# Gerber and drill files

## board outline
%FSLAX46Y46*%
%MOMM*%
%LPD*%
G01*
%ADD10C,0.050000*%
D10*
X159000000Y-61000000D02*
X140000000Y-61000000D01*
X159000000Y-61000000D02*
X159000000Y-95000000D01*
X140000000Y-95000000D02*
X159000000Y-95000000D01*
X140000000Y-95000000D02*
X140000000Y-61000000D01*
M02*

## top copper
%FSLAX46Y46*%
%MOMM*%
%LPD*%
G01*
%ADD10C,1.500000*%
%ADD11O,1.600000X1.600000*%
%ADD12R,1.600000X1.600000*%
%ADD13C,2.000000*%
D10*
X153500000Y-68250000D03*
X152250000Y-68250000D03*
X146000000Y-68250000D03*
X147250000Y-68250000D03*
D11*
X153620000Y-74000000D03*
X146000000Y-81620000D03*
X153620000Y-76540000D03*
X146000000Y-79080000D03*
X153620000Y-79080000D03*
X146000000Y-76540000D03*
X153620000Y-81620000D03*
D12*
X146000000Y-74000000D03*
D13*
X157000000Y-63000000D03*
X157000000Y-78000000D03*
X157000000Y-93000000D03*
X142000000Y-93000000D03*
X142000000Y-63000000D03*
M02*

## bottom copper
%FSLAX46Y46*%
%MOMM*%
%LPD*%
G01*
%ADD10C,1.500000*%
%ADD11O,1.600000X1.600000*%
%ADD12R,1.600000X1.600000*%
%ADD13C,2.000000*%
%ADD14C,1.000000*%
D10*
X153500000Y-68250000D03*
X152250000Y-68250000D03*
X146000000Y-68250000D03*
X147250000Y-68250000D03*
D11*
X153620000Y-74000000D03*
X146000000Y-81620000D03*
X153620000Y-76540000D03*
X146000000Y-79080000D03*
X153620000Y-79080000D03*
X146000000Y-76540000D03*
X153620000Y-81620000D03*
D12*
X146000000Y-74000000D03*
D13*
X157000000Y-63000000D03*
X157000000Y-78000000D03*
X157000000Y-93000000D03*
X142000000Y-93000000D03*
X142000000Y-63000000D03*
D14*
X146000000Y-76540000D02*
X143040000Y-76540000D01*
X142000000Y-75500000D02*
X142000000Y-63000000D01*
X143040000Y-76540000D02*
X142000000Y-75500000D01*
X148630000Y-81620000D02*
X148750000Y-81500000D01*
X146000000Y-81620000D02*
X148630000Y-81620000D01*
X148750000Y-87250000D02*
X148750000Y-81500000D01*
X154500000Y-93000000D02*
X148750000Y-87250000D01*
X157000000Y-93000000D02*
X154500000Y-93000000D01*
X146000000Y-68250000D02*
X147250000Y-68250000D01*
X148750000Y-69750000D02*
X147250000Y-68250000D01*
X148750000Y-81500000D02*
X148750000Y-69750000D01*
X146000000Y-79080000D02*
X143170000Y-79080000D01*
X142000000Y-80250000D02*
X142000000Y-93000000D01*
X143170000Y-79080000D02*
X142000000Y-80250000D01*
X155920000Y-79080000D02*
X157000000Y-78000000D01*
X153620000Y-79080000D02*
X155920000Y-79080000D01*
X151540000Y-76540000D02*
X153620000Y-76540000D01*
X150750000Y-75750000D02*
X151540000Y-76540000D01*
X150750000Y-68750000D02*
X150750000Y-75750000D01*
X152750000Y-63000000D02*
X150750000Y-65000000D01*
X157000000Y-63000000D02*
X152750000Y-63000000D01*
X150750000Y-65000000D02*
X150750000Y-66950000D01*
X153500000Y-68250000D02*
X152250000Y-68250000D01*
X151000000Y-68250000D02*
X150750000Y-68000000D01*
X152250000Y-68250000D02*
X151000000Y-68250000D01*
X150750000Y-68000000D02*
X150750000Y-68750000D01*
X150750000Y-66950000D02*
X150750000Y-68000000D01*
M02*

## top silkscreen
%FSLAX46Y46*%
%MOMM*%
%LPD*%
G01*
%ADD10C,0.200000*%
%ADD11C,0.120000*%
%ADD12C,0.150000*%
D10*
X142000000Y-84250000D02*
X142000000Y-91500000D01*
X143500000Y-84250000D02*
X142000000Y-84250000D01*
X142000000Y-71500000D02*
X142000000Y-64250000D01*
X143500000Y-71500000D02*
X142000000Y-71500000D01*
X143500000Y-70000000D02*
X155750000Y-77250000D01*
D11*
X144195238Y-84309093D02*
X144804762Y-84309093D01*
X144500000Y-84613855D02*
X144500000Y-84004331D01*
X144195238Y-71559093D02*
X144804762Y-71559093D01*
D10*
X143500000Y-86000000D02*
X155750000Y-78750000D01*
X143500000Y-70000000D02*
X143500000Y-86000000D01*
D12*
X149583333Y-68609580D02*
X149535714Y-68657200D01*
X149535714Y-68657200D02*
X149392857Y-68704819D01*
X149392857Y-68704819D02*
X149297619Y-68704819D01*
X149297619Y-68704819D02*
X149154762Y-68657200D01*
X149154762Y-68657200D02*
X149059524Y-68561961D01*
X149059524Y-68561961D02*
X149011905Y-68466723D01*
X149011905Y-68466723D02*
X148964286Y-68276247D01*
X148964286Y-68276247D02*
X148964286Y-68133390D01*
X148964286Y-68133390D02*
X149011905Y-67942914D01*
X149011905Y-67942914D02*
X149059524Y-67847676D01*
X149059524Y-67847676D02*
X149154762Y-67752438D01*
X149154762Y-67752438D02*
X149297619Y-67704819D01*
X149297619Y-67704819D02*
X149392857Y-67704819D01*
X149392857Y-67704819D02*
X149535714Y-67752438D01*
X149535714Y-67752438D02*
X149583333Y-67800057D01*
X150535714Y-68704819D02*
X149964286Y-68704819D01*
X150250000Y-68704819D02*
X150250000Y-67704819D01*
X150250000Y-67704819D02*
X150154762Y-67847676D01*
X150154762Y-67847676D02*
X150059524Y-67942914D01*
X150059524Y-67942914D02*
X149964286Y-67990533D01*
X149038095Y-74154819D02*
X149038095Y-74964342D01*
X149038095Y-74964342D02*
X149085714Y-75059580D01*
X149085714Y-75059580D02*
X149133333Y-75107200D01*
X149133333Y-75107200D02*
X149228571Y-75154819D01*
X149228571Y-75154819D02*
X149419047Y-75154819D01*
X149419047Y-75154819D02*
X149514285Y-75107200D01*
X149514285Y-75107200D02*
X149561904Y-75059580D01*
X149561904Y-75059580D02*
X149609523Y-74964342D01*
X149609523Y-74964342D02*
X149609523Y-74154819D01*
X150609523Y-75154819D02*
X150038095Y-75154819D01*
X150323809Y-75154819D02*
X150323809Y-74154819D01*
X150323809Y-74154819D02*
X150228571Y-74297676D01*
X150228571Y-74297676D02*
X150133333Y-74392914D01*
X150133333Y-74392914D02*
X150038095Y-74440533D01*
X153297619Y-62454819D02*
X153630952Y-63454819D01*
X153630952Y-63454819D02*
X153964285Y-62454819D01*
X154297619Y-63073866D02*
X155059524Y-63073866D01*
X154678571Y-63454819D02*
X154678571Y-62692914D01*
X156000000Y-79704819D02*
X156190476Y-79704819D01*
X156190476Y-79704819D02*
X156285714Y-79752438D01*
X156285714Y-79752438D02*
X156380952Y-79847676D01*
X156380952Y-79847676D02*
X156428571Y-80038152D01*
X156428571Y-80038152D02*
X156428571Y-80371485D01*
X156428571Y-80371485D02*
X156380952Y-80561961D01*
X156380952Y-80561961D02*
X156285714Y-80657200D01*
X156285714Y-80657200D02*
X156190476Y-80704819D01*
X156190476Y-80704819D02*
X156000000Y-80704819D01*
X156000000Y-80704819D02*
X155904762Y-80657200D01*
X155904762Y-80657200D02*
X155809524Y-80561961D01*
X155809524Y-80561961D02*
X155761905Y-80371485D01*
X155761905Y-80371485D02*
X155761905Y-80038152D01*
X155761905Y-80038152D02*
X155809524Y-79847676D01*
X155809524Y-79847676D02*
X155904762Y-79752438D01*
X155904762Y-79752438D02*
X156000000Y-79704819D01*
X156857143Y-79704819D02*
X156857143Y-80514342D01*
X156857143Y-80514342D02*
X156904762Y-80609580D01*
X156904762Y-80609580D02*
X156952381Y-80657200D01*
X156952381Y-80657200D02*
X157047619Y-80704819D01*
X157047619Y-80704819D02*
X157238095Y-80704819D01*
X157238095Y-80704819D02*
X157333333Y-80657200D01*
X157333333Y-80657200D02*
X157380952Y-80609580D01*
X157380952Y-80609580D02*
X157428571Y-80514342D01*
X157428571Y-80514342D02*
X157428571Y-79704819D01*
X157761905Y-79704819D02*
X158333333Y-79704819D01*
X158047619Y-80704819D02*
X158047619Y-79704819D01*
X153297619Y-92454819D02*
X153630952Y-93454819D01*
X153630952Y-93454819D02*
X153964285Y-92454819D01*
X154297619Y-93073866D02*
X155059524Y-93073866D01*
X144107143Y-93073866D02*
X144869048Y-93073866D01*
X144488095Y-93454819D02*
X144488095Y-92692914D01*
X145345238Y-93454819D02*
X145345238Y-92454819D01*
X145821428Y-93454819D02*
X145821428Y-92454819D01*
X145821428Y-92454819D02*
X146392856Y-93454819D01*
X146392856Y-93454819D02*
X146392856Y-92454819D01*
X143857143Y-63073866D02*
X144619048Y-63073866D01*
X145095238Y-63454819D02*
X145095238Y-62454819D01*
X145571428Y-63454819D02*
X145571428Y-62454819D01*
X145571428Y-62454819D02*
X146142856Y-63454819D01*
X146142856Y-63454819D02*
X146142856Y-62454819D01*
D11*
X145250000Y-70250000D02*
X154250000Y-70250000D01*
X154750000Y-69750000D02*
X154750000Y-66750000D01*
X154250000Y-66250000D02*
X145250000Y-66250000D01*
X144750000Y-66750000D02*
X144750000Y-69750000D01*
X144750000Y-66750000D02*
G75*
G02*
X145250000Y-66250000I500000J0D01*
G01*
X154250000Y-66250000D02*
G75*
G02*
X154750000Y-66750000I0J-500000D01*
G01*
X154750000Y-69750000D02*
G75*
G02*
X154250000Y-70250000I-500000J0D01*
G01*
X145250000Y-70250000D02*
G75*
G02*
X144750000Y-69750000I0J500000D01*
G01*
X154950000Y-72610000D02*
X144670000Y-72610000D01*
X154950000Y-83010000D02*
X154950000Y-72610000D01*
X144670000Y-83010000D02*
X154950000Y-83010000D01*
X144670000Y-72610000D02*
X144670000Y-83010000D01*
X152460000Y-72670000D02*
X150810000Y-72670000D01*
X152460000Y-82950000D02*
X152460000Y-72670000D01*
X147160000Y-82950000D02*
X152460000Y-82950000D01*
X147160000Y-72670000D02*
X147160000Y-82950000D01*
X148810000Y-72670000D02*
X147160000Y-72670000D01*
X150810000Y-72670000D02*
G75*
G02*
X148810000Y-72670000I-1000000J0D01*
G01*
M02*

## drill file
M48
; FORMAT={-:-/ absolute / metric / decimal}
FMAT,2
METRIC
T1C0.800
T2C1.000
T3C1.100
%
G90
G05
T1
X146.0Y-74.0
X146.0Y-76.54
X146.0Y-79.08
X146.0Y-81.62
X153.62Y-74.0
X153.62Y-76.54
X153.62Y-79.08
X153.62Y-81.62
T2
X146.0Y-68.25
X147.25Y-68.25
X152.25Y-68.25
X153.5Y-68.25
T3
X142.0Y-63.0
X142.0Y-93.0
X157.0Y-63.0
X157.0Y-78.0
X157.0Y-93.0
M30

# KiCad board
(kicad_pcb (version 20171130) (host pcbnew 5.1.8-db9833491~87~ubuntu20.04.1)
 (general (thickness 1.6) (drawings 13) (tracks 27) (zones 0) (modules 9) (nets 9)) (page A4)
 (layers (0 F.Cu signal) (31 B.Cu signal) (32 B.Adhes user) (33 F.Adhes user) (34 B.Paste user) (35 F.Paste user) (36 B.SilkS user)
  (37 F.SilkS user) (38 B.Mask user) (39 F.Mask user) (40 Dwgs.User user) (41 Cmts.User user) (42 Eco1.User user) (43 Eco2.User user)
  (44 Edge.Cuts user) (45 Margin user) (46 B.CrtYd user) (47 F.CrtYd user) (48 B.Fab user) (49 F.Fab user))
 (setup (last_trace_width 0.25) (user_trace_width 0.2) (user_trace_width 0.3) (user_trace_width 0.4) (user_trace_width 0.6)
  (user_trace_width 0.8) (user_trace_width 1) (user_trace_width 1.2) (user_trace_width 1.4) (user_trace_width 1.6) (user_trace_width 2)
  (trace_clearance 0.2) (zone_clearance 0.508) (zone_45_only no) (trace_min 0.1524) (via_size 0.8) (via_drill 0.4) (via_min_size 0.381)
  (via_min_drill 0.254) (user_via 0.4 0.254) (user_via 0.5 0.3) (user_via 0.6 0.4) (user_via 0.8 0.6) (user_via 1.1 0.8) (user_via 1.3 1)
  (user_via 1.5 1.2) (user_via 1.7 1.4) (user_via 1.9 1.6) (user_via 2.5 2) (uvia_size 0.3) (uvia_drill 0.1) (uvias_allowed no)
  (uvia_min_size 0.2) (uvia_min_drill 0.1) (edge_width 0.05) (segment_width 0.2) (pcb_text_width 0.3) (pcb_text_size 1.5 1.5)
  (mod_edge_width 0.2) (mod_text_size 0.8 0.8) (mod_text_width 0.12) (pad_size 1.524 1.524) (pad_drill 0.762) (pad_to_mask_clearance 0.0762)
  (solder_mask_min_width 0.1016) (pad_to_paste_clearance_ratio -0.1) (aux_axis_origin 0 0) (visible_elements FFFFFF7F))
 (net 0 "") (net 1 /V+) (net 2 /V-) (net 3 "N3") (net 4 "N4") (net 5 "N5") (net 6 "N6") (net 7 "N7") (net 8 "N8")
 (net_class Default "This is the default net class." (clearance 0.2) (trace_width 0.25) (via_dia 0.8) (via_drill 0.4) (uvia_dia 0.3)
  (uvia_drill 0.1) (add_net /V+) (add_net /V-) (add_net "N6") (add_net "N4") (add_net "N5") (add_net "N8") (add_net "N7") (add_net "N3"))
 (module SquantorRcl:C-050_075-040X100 (layer F.Cu) (at 149.75 68.25)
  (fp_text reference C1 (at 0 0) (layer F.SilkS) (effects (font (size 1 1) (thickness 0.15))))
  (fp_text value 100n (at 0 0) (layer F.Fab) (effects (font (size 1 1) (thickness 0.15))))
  (fp_line (start -4.5 2) (end 4.5 2) (layer F.SilkS) (width 0.12))
  (fp_line (start 5 1.5) (end 5 -1.5) (layer F.SilkS) (width 0.12))
  (fp_line (start 4.5 -2) (end -4.5 -2) (layer F.SilkS) (width 0.12))
  (fp_line (start -5 -1.5) (end -5 1.5) (layer F.SilkS) (width 0.12))
  (fp_arc (start -4.5 -1.5) (end -4.5 -2) (angle -90) (layer F.SilkS) (width 0.12))
  (fp_arc (start 4.5 -1.5) (end 5 -1.5) (angle -90) (layer F.SilkS) (width 0.12))
  (fp_arc (start 4.5 1.5) (end 4.5 2) (angle -90) (layer F.SilkS) (width 0.12))
  (fp_arc (start -4.5 1.5) (end -5 1.5) (angle -90) (layer F.SilkS) (width 0.12))
  (pad 2 thru_hole circle (at 3.75 0) (size 1.5 1.5) (drill 1) (layers *.Cu *.Mask) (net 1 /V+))
  (pad 2 thru_hole circle (at 2.5 0) (size 1.5 1.5) (drill 1) (layers *.Cu *.Mask) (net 1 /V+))
  (pad 1 thru_hole circle (at -3.75 0) (size 1.5 1.5) (drill 1) (layers *.Cu *.Mask) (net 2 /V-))
  (pad 1 thru_hole circle (at -2.5 0) (size 1.5 1.5) (drill 1) (layers *.Cu *.Mask) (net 2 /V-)))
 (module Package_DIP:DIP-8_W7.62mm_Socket (layer F.Cu) (at 146 74)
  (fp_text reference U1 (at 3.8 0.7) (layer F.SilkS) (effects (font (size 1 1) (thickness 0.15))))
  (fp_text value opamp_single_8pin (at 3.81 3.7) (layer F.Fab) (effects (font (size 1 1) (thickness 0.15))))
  (fp_line (start 8.95 -1.39) (end -1.33 -1.39) (layer F.SilkS) (width 0.12))
  (fp_line (start 8.95 9.01) (end 8.95 -1.39) (layer F.SilkS) (width 0.12))
  (fp_line (start -1.33 9.01) (end 8.95 9.01) (layer F.SilkS) (width 0.12))
  (fp_line (start -1.33 -1.39) (end -1.33 9.01) (layer F.SilkS) (width 0.12))
  (fp_line (start 6.46 -1.33) (end 4.81 -1.33) (layer F.SilkS) (width 0.12))
  (fp_line (start 6.46 8.95) (end 6.46 -1.33) (layer F.SilkS) (width 0.12))
  (fp_line (start 1.16 8.95) (end 6.46 8.95) (layer F.SilkS) (width 0.12))
  (fp_line (start 1.16 -1.33) (end 1.16 8.95) (layer F.SilkS) (width 0.12))
  (fp_line (start 2.81 -1.33) (end 1.16 -1.33) (layer F.SilkS) (width 0.12))
  (fp_arc (start 3.81 -1.33) (end 2.81 -1.33) (angle -180) (layer F.SilkS) (width 0.12))
  (pad 8 thru_hole oval (at 7.62 0) (size 1.6 1.6) (drill 0.8) (layers *.Cu *.Mask) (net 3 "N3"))
  (pad 4 thru_hole oval (at 0 7.62) (size 1.6 1.6) (drill 0.8) (layers *.Cu *.Mask) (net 2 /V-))
  (pad 7 thru_hole oval (at 7.62 2.54) (size 1.6 1.6) (drill 0.8) (layers *.Cu *.Mask) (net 1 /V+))
  (pad 3 thru_hole oval (at 0 5.08) (size 1.6 1.6) (drill 0.8) (layers *.Cu *.Mask) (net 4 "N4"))
  (pad 6 thru_hole oval (at 7.62 5.08) (size 1.6 1.6) (drill 0.8) (layers *.Cu *.Mask) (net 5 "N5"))
  (pad 2 thru_hole oval (at 0 2.54) (size 1.6 1.6) (drill 0.8) (layers *.Cu *.Mask) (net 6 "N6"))
  (pad 5 thru_hole oval (at 7.62 7.62) (size 1.6 1.6) (drill 0.8) (layers *.Cu *.Mask) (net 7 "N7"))
  (pad 1 thru_hole rect (at 0 0) (size 1.6 1.6) (drill 0.8) (layers *.Cu *.Mask) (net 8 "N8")))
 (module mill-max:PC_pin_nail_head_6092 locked (layer F.Cu) (at 157 63)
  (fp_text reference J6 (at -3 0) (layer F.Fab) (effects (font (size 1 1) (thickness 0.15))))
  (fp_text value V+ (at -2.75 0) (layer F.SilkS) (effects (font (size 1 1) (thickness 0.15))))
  (pad 1 thru_hole circle (at 0 0) (size 2 2) (drill 1.1) (layers *.Cu *.Mask) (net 1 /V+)))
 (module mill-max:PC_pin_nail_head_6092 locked (layer F.Cu) (at 157 78)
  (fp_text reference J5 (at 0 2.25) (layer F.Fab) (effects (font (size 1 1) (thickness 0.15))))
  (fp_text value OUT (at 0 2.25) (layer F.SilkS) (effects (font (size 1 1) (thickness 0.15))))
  (pad 1 thru_hole circle (at 0 0) (size 2 2) (drill 1.1) (layers *.Cu *.Mask) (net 5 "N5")))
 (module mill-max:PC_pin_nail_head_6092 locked (layer F.Cu) (at 157 93)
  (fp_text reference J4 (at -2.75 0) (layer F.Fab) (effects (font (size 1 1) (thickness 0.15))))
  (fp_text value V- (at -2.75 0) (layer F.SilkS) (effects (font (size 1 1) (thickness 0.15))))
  (pad 1 thru_hole circle (at 0 0) (size 2 2) (drill 1.1) (layers *.Cu *.Mask) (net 2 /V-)))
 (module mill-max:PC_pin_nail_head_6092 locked (layer F.Cu) (at 142 93)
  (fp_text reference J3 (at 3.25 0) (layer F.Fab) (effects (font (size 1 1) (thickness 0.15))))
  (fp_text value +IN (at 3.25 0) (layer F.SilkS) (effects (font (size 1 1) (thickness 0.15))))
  (pad 1 thru_hole circle (at 0 0) (size 2 2) (drill 1.1) (layers *.Cu *.Mask) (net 4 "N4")))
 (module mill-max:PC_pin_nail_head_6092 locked (layer F.Cu) (at 142 63)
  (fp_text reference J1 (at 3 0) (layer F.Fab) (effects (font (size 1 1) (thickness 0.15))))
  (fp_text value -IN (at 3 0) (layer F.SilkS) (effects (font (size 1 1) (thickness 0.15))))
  (pad 1 thru_hole circle (at 0 0) (size 2 2) (drill 1.1) (layers *.Cu *.Mask) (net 6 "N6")))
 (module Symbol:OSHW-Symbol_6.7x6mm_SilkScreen (layer B.Cu) (at 150 86.25 180)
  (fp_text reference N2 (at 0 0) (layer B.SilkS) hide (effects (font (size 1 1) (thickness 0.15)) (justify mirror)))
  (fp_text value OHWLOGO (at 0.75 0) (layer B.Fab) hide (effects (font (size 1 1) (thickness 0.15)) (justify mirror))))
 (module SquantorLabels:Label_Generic (layer B.Cu) (at 149.25 90)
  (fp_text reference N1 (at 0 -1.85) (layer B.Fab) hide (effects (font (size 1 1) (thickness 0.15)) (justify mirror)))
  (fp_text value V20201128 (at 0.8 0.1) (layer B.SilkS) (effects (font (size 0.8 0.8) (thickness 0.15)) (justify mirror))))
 (gr_line (start 142 84.25) (end 142 91.5) (layer F.SilkS) (width 0.2))
 (gr_line (start 143.5 84.25) (end 142 84.25) (layer F.SilkS) (width 0.2))
 (gr_line (start 142 71.5) (end 142 64.25) (layer F.SilkS) (width 0.2))
 (gr_line (start 143.5 71.5) (end 142 71.5) (layer F.SilkS) (width 0.2))
 (gr_line (start 143.5 70) (end 155.75 77.25) (layer F.SilkS) (width 0.2))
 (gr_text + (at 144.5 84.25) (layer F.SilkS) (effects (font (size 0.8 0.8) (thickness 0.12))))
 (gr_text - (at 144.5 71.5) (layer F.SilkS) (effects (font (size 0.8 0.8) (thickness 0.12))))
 (gr_line (start 143.5 86) (end 155.75 78.75) (layer F.SilkS) (width 0.2))
 (gr_line (start 143.5 70) (end 143.5 86) (layer F.SilkS) (width 0.2))
 (gr_line (start 159 61) (end 140 61) (layer Edge.Cuts) (width 0.05))
 (gr_line (start 159 61) (end 159 95) (layer Edge.Cuts) (width 0.05))
 (gr_line (start 140 95) (end 159 95) (layer Edge.Cuts) (width 0.05))
 (gr_line (start 140 95) (end 140 61) (layer Edge.Cuts) (width 0.05))
 (segment (start 146 76.54) (end 143.04 76.54) (width 1) (layer B.Cu) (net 6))
 (segment (start 142 75.5) (end 142 63) (width 1) (layer B.Cu) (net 6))
 (segment (start 143.04 76.54) (end 142 75.5) (width 1) (layer B.Cu) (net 6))
 (segment (start 148.63 81.62) (end 148.75 81.5) (width 1) (layer B.Cu) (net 2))
 (segment (start 146 81.62) (end 148.63 81.62) (width 1) (layer B.Cu) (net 2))
 (segment (start 148.75 87.25) (end 148.75 81.5) (width 1) (layer B.Cu) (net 2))
 (segment (start 154.5 93) (end 148.75 87.25) (width 1) (layer B.Cu) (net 2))
 (segment (start 157 93) (end 154.5 93) (width 1) (layer B.Cu) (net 2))
 (segment (start 146 68.25) (end 147.25 68.25) (width 1) (layer B.Cu) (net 2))
 (segment (start 148.75 69.75) (end 147.25 68.25) (width 1) (layer B.Cu) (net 2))
 (segment (start 148.75 81.5) (end 148.75 69.75) (width 1) (layer B.Cu) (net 2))
 (segment (start 146 79.08) (end 143.17 79.08) (width 1) (layer B.Cu) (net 4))
 (segment (start 142 80.25) (end 142 93) (width 1) (layer B.Cu) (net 4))
 (segment (start 143.17 79.08) (end 142 80.25) (width 1) (layer B.Cu) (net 4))
 (segment (start 155.92 79.08) (end 157 78) (width 1) (layer B.Cu) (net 5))
 (segment (start 153.62 79.08) (end 155.92 79.08) (width 1) (layer B.Cu) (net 5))
 (segment (start 151.54 76.54) (end 153.62 76.54) (width 1) (layer B.Cu) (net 1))
 (segment (start 150.75 75.75) (end 151.54 76.54) (width 1) (layer B.Cu) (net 1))
 (segment (start 150.75 68.75) (end 150.75 75.75) (width 1) (layer B.Cu) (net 1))
 (segment (start 152.75 63) (end 150.75 65) (width 1) (layer B.Cu) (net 1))
 (segment (start 157 63) (end 152.75 63) (width 1) (layer B.Cu) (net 1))
 (segment (start 150.75 65) (end 150.75 66.95) (width 1) (layer B.Cu) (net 1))
 (segment (start 153.5 68.25) (end 152.25 68.25) (width 1) (layer B.Cu) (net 1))
 (segment (start 151 68.25) (end 150.75 68) (width 1) (layer B.Cu) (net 1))
 (segment (start 152.25 68.25) (end 151 68.25) (width 1) (layer B.Cu) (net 1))
 (segment (start 150.75 68) (end 150.75 68.75) (width 1) (layer B.Cu) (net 1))
 (segment (start 150.75 66.95) (end 150.75 68) (width 1) (layer B.Cu) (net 1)))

